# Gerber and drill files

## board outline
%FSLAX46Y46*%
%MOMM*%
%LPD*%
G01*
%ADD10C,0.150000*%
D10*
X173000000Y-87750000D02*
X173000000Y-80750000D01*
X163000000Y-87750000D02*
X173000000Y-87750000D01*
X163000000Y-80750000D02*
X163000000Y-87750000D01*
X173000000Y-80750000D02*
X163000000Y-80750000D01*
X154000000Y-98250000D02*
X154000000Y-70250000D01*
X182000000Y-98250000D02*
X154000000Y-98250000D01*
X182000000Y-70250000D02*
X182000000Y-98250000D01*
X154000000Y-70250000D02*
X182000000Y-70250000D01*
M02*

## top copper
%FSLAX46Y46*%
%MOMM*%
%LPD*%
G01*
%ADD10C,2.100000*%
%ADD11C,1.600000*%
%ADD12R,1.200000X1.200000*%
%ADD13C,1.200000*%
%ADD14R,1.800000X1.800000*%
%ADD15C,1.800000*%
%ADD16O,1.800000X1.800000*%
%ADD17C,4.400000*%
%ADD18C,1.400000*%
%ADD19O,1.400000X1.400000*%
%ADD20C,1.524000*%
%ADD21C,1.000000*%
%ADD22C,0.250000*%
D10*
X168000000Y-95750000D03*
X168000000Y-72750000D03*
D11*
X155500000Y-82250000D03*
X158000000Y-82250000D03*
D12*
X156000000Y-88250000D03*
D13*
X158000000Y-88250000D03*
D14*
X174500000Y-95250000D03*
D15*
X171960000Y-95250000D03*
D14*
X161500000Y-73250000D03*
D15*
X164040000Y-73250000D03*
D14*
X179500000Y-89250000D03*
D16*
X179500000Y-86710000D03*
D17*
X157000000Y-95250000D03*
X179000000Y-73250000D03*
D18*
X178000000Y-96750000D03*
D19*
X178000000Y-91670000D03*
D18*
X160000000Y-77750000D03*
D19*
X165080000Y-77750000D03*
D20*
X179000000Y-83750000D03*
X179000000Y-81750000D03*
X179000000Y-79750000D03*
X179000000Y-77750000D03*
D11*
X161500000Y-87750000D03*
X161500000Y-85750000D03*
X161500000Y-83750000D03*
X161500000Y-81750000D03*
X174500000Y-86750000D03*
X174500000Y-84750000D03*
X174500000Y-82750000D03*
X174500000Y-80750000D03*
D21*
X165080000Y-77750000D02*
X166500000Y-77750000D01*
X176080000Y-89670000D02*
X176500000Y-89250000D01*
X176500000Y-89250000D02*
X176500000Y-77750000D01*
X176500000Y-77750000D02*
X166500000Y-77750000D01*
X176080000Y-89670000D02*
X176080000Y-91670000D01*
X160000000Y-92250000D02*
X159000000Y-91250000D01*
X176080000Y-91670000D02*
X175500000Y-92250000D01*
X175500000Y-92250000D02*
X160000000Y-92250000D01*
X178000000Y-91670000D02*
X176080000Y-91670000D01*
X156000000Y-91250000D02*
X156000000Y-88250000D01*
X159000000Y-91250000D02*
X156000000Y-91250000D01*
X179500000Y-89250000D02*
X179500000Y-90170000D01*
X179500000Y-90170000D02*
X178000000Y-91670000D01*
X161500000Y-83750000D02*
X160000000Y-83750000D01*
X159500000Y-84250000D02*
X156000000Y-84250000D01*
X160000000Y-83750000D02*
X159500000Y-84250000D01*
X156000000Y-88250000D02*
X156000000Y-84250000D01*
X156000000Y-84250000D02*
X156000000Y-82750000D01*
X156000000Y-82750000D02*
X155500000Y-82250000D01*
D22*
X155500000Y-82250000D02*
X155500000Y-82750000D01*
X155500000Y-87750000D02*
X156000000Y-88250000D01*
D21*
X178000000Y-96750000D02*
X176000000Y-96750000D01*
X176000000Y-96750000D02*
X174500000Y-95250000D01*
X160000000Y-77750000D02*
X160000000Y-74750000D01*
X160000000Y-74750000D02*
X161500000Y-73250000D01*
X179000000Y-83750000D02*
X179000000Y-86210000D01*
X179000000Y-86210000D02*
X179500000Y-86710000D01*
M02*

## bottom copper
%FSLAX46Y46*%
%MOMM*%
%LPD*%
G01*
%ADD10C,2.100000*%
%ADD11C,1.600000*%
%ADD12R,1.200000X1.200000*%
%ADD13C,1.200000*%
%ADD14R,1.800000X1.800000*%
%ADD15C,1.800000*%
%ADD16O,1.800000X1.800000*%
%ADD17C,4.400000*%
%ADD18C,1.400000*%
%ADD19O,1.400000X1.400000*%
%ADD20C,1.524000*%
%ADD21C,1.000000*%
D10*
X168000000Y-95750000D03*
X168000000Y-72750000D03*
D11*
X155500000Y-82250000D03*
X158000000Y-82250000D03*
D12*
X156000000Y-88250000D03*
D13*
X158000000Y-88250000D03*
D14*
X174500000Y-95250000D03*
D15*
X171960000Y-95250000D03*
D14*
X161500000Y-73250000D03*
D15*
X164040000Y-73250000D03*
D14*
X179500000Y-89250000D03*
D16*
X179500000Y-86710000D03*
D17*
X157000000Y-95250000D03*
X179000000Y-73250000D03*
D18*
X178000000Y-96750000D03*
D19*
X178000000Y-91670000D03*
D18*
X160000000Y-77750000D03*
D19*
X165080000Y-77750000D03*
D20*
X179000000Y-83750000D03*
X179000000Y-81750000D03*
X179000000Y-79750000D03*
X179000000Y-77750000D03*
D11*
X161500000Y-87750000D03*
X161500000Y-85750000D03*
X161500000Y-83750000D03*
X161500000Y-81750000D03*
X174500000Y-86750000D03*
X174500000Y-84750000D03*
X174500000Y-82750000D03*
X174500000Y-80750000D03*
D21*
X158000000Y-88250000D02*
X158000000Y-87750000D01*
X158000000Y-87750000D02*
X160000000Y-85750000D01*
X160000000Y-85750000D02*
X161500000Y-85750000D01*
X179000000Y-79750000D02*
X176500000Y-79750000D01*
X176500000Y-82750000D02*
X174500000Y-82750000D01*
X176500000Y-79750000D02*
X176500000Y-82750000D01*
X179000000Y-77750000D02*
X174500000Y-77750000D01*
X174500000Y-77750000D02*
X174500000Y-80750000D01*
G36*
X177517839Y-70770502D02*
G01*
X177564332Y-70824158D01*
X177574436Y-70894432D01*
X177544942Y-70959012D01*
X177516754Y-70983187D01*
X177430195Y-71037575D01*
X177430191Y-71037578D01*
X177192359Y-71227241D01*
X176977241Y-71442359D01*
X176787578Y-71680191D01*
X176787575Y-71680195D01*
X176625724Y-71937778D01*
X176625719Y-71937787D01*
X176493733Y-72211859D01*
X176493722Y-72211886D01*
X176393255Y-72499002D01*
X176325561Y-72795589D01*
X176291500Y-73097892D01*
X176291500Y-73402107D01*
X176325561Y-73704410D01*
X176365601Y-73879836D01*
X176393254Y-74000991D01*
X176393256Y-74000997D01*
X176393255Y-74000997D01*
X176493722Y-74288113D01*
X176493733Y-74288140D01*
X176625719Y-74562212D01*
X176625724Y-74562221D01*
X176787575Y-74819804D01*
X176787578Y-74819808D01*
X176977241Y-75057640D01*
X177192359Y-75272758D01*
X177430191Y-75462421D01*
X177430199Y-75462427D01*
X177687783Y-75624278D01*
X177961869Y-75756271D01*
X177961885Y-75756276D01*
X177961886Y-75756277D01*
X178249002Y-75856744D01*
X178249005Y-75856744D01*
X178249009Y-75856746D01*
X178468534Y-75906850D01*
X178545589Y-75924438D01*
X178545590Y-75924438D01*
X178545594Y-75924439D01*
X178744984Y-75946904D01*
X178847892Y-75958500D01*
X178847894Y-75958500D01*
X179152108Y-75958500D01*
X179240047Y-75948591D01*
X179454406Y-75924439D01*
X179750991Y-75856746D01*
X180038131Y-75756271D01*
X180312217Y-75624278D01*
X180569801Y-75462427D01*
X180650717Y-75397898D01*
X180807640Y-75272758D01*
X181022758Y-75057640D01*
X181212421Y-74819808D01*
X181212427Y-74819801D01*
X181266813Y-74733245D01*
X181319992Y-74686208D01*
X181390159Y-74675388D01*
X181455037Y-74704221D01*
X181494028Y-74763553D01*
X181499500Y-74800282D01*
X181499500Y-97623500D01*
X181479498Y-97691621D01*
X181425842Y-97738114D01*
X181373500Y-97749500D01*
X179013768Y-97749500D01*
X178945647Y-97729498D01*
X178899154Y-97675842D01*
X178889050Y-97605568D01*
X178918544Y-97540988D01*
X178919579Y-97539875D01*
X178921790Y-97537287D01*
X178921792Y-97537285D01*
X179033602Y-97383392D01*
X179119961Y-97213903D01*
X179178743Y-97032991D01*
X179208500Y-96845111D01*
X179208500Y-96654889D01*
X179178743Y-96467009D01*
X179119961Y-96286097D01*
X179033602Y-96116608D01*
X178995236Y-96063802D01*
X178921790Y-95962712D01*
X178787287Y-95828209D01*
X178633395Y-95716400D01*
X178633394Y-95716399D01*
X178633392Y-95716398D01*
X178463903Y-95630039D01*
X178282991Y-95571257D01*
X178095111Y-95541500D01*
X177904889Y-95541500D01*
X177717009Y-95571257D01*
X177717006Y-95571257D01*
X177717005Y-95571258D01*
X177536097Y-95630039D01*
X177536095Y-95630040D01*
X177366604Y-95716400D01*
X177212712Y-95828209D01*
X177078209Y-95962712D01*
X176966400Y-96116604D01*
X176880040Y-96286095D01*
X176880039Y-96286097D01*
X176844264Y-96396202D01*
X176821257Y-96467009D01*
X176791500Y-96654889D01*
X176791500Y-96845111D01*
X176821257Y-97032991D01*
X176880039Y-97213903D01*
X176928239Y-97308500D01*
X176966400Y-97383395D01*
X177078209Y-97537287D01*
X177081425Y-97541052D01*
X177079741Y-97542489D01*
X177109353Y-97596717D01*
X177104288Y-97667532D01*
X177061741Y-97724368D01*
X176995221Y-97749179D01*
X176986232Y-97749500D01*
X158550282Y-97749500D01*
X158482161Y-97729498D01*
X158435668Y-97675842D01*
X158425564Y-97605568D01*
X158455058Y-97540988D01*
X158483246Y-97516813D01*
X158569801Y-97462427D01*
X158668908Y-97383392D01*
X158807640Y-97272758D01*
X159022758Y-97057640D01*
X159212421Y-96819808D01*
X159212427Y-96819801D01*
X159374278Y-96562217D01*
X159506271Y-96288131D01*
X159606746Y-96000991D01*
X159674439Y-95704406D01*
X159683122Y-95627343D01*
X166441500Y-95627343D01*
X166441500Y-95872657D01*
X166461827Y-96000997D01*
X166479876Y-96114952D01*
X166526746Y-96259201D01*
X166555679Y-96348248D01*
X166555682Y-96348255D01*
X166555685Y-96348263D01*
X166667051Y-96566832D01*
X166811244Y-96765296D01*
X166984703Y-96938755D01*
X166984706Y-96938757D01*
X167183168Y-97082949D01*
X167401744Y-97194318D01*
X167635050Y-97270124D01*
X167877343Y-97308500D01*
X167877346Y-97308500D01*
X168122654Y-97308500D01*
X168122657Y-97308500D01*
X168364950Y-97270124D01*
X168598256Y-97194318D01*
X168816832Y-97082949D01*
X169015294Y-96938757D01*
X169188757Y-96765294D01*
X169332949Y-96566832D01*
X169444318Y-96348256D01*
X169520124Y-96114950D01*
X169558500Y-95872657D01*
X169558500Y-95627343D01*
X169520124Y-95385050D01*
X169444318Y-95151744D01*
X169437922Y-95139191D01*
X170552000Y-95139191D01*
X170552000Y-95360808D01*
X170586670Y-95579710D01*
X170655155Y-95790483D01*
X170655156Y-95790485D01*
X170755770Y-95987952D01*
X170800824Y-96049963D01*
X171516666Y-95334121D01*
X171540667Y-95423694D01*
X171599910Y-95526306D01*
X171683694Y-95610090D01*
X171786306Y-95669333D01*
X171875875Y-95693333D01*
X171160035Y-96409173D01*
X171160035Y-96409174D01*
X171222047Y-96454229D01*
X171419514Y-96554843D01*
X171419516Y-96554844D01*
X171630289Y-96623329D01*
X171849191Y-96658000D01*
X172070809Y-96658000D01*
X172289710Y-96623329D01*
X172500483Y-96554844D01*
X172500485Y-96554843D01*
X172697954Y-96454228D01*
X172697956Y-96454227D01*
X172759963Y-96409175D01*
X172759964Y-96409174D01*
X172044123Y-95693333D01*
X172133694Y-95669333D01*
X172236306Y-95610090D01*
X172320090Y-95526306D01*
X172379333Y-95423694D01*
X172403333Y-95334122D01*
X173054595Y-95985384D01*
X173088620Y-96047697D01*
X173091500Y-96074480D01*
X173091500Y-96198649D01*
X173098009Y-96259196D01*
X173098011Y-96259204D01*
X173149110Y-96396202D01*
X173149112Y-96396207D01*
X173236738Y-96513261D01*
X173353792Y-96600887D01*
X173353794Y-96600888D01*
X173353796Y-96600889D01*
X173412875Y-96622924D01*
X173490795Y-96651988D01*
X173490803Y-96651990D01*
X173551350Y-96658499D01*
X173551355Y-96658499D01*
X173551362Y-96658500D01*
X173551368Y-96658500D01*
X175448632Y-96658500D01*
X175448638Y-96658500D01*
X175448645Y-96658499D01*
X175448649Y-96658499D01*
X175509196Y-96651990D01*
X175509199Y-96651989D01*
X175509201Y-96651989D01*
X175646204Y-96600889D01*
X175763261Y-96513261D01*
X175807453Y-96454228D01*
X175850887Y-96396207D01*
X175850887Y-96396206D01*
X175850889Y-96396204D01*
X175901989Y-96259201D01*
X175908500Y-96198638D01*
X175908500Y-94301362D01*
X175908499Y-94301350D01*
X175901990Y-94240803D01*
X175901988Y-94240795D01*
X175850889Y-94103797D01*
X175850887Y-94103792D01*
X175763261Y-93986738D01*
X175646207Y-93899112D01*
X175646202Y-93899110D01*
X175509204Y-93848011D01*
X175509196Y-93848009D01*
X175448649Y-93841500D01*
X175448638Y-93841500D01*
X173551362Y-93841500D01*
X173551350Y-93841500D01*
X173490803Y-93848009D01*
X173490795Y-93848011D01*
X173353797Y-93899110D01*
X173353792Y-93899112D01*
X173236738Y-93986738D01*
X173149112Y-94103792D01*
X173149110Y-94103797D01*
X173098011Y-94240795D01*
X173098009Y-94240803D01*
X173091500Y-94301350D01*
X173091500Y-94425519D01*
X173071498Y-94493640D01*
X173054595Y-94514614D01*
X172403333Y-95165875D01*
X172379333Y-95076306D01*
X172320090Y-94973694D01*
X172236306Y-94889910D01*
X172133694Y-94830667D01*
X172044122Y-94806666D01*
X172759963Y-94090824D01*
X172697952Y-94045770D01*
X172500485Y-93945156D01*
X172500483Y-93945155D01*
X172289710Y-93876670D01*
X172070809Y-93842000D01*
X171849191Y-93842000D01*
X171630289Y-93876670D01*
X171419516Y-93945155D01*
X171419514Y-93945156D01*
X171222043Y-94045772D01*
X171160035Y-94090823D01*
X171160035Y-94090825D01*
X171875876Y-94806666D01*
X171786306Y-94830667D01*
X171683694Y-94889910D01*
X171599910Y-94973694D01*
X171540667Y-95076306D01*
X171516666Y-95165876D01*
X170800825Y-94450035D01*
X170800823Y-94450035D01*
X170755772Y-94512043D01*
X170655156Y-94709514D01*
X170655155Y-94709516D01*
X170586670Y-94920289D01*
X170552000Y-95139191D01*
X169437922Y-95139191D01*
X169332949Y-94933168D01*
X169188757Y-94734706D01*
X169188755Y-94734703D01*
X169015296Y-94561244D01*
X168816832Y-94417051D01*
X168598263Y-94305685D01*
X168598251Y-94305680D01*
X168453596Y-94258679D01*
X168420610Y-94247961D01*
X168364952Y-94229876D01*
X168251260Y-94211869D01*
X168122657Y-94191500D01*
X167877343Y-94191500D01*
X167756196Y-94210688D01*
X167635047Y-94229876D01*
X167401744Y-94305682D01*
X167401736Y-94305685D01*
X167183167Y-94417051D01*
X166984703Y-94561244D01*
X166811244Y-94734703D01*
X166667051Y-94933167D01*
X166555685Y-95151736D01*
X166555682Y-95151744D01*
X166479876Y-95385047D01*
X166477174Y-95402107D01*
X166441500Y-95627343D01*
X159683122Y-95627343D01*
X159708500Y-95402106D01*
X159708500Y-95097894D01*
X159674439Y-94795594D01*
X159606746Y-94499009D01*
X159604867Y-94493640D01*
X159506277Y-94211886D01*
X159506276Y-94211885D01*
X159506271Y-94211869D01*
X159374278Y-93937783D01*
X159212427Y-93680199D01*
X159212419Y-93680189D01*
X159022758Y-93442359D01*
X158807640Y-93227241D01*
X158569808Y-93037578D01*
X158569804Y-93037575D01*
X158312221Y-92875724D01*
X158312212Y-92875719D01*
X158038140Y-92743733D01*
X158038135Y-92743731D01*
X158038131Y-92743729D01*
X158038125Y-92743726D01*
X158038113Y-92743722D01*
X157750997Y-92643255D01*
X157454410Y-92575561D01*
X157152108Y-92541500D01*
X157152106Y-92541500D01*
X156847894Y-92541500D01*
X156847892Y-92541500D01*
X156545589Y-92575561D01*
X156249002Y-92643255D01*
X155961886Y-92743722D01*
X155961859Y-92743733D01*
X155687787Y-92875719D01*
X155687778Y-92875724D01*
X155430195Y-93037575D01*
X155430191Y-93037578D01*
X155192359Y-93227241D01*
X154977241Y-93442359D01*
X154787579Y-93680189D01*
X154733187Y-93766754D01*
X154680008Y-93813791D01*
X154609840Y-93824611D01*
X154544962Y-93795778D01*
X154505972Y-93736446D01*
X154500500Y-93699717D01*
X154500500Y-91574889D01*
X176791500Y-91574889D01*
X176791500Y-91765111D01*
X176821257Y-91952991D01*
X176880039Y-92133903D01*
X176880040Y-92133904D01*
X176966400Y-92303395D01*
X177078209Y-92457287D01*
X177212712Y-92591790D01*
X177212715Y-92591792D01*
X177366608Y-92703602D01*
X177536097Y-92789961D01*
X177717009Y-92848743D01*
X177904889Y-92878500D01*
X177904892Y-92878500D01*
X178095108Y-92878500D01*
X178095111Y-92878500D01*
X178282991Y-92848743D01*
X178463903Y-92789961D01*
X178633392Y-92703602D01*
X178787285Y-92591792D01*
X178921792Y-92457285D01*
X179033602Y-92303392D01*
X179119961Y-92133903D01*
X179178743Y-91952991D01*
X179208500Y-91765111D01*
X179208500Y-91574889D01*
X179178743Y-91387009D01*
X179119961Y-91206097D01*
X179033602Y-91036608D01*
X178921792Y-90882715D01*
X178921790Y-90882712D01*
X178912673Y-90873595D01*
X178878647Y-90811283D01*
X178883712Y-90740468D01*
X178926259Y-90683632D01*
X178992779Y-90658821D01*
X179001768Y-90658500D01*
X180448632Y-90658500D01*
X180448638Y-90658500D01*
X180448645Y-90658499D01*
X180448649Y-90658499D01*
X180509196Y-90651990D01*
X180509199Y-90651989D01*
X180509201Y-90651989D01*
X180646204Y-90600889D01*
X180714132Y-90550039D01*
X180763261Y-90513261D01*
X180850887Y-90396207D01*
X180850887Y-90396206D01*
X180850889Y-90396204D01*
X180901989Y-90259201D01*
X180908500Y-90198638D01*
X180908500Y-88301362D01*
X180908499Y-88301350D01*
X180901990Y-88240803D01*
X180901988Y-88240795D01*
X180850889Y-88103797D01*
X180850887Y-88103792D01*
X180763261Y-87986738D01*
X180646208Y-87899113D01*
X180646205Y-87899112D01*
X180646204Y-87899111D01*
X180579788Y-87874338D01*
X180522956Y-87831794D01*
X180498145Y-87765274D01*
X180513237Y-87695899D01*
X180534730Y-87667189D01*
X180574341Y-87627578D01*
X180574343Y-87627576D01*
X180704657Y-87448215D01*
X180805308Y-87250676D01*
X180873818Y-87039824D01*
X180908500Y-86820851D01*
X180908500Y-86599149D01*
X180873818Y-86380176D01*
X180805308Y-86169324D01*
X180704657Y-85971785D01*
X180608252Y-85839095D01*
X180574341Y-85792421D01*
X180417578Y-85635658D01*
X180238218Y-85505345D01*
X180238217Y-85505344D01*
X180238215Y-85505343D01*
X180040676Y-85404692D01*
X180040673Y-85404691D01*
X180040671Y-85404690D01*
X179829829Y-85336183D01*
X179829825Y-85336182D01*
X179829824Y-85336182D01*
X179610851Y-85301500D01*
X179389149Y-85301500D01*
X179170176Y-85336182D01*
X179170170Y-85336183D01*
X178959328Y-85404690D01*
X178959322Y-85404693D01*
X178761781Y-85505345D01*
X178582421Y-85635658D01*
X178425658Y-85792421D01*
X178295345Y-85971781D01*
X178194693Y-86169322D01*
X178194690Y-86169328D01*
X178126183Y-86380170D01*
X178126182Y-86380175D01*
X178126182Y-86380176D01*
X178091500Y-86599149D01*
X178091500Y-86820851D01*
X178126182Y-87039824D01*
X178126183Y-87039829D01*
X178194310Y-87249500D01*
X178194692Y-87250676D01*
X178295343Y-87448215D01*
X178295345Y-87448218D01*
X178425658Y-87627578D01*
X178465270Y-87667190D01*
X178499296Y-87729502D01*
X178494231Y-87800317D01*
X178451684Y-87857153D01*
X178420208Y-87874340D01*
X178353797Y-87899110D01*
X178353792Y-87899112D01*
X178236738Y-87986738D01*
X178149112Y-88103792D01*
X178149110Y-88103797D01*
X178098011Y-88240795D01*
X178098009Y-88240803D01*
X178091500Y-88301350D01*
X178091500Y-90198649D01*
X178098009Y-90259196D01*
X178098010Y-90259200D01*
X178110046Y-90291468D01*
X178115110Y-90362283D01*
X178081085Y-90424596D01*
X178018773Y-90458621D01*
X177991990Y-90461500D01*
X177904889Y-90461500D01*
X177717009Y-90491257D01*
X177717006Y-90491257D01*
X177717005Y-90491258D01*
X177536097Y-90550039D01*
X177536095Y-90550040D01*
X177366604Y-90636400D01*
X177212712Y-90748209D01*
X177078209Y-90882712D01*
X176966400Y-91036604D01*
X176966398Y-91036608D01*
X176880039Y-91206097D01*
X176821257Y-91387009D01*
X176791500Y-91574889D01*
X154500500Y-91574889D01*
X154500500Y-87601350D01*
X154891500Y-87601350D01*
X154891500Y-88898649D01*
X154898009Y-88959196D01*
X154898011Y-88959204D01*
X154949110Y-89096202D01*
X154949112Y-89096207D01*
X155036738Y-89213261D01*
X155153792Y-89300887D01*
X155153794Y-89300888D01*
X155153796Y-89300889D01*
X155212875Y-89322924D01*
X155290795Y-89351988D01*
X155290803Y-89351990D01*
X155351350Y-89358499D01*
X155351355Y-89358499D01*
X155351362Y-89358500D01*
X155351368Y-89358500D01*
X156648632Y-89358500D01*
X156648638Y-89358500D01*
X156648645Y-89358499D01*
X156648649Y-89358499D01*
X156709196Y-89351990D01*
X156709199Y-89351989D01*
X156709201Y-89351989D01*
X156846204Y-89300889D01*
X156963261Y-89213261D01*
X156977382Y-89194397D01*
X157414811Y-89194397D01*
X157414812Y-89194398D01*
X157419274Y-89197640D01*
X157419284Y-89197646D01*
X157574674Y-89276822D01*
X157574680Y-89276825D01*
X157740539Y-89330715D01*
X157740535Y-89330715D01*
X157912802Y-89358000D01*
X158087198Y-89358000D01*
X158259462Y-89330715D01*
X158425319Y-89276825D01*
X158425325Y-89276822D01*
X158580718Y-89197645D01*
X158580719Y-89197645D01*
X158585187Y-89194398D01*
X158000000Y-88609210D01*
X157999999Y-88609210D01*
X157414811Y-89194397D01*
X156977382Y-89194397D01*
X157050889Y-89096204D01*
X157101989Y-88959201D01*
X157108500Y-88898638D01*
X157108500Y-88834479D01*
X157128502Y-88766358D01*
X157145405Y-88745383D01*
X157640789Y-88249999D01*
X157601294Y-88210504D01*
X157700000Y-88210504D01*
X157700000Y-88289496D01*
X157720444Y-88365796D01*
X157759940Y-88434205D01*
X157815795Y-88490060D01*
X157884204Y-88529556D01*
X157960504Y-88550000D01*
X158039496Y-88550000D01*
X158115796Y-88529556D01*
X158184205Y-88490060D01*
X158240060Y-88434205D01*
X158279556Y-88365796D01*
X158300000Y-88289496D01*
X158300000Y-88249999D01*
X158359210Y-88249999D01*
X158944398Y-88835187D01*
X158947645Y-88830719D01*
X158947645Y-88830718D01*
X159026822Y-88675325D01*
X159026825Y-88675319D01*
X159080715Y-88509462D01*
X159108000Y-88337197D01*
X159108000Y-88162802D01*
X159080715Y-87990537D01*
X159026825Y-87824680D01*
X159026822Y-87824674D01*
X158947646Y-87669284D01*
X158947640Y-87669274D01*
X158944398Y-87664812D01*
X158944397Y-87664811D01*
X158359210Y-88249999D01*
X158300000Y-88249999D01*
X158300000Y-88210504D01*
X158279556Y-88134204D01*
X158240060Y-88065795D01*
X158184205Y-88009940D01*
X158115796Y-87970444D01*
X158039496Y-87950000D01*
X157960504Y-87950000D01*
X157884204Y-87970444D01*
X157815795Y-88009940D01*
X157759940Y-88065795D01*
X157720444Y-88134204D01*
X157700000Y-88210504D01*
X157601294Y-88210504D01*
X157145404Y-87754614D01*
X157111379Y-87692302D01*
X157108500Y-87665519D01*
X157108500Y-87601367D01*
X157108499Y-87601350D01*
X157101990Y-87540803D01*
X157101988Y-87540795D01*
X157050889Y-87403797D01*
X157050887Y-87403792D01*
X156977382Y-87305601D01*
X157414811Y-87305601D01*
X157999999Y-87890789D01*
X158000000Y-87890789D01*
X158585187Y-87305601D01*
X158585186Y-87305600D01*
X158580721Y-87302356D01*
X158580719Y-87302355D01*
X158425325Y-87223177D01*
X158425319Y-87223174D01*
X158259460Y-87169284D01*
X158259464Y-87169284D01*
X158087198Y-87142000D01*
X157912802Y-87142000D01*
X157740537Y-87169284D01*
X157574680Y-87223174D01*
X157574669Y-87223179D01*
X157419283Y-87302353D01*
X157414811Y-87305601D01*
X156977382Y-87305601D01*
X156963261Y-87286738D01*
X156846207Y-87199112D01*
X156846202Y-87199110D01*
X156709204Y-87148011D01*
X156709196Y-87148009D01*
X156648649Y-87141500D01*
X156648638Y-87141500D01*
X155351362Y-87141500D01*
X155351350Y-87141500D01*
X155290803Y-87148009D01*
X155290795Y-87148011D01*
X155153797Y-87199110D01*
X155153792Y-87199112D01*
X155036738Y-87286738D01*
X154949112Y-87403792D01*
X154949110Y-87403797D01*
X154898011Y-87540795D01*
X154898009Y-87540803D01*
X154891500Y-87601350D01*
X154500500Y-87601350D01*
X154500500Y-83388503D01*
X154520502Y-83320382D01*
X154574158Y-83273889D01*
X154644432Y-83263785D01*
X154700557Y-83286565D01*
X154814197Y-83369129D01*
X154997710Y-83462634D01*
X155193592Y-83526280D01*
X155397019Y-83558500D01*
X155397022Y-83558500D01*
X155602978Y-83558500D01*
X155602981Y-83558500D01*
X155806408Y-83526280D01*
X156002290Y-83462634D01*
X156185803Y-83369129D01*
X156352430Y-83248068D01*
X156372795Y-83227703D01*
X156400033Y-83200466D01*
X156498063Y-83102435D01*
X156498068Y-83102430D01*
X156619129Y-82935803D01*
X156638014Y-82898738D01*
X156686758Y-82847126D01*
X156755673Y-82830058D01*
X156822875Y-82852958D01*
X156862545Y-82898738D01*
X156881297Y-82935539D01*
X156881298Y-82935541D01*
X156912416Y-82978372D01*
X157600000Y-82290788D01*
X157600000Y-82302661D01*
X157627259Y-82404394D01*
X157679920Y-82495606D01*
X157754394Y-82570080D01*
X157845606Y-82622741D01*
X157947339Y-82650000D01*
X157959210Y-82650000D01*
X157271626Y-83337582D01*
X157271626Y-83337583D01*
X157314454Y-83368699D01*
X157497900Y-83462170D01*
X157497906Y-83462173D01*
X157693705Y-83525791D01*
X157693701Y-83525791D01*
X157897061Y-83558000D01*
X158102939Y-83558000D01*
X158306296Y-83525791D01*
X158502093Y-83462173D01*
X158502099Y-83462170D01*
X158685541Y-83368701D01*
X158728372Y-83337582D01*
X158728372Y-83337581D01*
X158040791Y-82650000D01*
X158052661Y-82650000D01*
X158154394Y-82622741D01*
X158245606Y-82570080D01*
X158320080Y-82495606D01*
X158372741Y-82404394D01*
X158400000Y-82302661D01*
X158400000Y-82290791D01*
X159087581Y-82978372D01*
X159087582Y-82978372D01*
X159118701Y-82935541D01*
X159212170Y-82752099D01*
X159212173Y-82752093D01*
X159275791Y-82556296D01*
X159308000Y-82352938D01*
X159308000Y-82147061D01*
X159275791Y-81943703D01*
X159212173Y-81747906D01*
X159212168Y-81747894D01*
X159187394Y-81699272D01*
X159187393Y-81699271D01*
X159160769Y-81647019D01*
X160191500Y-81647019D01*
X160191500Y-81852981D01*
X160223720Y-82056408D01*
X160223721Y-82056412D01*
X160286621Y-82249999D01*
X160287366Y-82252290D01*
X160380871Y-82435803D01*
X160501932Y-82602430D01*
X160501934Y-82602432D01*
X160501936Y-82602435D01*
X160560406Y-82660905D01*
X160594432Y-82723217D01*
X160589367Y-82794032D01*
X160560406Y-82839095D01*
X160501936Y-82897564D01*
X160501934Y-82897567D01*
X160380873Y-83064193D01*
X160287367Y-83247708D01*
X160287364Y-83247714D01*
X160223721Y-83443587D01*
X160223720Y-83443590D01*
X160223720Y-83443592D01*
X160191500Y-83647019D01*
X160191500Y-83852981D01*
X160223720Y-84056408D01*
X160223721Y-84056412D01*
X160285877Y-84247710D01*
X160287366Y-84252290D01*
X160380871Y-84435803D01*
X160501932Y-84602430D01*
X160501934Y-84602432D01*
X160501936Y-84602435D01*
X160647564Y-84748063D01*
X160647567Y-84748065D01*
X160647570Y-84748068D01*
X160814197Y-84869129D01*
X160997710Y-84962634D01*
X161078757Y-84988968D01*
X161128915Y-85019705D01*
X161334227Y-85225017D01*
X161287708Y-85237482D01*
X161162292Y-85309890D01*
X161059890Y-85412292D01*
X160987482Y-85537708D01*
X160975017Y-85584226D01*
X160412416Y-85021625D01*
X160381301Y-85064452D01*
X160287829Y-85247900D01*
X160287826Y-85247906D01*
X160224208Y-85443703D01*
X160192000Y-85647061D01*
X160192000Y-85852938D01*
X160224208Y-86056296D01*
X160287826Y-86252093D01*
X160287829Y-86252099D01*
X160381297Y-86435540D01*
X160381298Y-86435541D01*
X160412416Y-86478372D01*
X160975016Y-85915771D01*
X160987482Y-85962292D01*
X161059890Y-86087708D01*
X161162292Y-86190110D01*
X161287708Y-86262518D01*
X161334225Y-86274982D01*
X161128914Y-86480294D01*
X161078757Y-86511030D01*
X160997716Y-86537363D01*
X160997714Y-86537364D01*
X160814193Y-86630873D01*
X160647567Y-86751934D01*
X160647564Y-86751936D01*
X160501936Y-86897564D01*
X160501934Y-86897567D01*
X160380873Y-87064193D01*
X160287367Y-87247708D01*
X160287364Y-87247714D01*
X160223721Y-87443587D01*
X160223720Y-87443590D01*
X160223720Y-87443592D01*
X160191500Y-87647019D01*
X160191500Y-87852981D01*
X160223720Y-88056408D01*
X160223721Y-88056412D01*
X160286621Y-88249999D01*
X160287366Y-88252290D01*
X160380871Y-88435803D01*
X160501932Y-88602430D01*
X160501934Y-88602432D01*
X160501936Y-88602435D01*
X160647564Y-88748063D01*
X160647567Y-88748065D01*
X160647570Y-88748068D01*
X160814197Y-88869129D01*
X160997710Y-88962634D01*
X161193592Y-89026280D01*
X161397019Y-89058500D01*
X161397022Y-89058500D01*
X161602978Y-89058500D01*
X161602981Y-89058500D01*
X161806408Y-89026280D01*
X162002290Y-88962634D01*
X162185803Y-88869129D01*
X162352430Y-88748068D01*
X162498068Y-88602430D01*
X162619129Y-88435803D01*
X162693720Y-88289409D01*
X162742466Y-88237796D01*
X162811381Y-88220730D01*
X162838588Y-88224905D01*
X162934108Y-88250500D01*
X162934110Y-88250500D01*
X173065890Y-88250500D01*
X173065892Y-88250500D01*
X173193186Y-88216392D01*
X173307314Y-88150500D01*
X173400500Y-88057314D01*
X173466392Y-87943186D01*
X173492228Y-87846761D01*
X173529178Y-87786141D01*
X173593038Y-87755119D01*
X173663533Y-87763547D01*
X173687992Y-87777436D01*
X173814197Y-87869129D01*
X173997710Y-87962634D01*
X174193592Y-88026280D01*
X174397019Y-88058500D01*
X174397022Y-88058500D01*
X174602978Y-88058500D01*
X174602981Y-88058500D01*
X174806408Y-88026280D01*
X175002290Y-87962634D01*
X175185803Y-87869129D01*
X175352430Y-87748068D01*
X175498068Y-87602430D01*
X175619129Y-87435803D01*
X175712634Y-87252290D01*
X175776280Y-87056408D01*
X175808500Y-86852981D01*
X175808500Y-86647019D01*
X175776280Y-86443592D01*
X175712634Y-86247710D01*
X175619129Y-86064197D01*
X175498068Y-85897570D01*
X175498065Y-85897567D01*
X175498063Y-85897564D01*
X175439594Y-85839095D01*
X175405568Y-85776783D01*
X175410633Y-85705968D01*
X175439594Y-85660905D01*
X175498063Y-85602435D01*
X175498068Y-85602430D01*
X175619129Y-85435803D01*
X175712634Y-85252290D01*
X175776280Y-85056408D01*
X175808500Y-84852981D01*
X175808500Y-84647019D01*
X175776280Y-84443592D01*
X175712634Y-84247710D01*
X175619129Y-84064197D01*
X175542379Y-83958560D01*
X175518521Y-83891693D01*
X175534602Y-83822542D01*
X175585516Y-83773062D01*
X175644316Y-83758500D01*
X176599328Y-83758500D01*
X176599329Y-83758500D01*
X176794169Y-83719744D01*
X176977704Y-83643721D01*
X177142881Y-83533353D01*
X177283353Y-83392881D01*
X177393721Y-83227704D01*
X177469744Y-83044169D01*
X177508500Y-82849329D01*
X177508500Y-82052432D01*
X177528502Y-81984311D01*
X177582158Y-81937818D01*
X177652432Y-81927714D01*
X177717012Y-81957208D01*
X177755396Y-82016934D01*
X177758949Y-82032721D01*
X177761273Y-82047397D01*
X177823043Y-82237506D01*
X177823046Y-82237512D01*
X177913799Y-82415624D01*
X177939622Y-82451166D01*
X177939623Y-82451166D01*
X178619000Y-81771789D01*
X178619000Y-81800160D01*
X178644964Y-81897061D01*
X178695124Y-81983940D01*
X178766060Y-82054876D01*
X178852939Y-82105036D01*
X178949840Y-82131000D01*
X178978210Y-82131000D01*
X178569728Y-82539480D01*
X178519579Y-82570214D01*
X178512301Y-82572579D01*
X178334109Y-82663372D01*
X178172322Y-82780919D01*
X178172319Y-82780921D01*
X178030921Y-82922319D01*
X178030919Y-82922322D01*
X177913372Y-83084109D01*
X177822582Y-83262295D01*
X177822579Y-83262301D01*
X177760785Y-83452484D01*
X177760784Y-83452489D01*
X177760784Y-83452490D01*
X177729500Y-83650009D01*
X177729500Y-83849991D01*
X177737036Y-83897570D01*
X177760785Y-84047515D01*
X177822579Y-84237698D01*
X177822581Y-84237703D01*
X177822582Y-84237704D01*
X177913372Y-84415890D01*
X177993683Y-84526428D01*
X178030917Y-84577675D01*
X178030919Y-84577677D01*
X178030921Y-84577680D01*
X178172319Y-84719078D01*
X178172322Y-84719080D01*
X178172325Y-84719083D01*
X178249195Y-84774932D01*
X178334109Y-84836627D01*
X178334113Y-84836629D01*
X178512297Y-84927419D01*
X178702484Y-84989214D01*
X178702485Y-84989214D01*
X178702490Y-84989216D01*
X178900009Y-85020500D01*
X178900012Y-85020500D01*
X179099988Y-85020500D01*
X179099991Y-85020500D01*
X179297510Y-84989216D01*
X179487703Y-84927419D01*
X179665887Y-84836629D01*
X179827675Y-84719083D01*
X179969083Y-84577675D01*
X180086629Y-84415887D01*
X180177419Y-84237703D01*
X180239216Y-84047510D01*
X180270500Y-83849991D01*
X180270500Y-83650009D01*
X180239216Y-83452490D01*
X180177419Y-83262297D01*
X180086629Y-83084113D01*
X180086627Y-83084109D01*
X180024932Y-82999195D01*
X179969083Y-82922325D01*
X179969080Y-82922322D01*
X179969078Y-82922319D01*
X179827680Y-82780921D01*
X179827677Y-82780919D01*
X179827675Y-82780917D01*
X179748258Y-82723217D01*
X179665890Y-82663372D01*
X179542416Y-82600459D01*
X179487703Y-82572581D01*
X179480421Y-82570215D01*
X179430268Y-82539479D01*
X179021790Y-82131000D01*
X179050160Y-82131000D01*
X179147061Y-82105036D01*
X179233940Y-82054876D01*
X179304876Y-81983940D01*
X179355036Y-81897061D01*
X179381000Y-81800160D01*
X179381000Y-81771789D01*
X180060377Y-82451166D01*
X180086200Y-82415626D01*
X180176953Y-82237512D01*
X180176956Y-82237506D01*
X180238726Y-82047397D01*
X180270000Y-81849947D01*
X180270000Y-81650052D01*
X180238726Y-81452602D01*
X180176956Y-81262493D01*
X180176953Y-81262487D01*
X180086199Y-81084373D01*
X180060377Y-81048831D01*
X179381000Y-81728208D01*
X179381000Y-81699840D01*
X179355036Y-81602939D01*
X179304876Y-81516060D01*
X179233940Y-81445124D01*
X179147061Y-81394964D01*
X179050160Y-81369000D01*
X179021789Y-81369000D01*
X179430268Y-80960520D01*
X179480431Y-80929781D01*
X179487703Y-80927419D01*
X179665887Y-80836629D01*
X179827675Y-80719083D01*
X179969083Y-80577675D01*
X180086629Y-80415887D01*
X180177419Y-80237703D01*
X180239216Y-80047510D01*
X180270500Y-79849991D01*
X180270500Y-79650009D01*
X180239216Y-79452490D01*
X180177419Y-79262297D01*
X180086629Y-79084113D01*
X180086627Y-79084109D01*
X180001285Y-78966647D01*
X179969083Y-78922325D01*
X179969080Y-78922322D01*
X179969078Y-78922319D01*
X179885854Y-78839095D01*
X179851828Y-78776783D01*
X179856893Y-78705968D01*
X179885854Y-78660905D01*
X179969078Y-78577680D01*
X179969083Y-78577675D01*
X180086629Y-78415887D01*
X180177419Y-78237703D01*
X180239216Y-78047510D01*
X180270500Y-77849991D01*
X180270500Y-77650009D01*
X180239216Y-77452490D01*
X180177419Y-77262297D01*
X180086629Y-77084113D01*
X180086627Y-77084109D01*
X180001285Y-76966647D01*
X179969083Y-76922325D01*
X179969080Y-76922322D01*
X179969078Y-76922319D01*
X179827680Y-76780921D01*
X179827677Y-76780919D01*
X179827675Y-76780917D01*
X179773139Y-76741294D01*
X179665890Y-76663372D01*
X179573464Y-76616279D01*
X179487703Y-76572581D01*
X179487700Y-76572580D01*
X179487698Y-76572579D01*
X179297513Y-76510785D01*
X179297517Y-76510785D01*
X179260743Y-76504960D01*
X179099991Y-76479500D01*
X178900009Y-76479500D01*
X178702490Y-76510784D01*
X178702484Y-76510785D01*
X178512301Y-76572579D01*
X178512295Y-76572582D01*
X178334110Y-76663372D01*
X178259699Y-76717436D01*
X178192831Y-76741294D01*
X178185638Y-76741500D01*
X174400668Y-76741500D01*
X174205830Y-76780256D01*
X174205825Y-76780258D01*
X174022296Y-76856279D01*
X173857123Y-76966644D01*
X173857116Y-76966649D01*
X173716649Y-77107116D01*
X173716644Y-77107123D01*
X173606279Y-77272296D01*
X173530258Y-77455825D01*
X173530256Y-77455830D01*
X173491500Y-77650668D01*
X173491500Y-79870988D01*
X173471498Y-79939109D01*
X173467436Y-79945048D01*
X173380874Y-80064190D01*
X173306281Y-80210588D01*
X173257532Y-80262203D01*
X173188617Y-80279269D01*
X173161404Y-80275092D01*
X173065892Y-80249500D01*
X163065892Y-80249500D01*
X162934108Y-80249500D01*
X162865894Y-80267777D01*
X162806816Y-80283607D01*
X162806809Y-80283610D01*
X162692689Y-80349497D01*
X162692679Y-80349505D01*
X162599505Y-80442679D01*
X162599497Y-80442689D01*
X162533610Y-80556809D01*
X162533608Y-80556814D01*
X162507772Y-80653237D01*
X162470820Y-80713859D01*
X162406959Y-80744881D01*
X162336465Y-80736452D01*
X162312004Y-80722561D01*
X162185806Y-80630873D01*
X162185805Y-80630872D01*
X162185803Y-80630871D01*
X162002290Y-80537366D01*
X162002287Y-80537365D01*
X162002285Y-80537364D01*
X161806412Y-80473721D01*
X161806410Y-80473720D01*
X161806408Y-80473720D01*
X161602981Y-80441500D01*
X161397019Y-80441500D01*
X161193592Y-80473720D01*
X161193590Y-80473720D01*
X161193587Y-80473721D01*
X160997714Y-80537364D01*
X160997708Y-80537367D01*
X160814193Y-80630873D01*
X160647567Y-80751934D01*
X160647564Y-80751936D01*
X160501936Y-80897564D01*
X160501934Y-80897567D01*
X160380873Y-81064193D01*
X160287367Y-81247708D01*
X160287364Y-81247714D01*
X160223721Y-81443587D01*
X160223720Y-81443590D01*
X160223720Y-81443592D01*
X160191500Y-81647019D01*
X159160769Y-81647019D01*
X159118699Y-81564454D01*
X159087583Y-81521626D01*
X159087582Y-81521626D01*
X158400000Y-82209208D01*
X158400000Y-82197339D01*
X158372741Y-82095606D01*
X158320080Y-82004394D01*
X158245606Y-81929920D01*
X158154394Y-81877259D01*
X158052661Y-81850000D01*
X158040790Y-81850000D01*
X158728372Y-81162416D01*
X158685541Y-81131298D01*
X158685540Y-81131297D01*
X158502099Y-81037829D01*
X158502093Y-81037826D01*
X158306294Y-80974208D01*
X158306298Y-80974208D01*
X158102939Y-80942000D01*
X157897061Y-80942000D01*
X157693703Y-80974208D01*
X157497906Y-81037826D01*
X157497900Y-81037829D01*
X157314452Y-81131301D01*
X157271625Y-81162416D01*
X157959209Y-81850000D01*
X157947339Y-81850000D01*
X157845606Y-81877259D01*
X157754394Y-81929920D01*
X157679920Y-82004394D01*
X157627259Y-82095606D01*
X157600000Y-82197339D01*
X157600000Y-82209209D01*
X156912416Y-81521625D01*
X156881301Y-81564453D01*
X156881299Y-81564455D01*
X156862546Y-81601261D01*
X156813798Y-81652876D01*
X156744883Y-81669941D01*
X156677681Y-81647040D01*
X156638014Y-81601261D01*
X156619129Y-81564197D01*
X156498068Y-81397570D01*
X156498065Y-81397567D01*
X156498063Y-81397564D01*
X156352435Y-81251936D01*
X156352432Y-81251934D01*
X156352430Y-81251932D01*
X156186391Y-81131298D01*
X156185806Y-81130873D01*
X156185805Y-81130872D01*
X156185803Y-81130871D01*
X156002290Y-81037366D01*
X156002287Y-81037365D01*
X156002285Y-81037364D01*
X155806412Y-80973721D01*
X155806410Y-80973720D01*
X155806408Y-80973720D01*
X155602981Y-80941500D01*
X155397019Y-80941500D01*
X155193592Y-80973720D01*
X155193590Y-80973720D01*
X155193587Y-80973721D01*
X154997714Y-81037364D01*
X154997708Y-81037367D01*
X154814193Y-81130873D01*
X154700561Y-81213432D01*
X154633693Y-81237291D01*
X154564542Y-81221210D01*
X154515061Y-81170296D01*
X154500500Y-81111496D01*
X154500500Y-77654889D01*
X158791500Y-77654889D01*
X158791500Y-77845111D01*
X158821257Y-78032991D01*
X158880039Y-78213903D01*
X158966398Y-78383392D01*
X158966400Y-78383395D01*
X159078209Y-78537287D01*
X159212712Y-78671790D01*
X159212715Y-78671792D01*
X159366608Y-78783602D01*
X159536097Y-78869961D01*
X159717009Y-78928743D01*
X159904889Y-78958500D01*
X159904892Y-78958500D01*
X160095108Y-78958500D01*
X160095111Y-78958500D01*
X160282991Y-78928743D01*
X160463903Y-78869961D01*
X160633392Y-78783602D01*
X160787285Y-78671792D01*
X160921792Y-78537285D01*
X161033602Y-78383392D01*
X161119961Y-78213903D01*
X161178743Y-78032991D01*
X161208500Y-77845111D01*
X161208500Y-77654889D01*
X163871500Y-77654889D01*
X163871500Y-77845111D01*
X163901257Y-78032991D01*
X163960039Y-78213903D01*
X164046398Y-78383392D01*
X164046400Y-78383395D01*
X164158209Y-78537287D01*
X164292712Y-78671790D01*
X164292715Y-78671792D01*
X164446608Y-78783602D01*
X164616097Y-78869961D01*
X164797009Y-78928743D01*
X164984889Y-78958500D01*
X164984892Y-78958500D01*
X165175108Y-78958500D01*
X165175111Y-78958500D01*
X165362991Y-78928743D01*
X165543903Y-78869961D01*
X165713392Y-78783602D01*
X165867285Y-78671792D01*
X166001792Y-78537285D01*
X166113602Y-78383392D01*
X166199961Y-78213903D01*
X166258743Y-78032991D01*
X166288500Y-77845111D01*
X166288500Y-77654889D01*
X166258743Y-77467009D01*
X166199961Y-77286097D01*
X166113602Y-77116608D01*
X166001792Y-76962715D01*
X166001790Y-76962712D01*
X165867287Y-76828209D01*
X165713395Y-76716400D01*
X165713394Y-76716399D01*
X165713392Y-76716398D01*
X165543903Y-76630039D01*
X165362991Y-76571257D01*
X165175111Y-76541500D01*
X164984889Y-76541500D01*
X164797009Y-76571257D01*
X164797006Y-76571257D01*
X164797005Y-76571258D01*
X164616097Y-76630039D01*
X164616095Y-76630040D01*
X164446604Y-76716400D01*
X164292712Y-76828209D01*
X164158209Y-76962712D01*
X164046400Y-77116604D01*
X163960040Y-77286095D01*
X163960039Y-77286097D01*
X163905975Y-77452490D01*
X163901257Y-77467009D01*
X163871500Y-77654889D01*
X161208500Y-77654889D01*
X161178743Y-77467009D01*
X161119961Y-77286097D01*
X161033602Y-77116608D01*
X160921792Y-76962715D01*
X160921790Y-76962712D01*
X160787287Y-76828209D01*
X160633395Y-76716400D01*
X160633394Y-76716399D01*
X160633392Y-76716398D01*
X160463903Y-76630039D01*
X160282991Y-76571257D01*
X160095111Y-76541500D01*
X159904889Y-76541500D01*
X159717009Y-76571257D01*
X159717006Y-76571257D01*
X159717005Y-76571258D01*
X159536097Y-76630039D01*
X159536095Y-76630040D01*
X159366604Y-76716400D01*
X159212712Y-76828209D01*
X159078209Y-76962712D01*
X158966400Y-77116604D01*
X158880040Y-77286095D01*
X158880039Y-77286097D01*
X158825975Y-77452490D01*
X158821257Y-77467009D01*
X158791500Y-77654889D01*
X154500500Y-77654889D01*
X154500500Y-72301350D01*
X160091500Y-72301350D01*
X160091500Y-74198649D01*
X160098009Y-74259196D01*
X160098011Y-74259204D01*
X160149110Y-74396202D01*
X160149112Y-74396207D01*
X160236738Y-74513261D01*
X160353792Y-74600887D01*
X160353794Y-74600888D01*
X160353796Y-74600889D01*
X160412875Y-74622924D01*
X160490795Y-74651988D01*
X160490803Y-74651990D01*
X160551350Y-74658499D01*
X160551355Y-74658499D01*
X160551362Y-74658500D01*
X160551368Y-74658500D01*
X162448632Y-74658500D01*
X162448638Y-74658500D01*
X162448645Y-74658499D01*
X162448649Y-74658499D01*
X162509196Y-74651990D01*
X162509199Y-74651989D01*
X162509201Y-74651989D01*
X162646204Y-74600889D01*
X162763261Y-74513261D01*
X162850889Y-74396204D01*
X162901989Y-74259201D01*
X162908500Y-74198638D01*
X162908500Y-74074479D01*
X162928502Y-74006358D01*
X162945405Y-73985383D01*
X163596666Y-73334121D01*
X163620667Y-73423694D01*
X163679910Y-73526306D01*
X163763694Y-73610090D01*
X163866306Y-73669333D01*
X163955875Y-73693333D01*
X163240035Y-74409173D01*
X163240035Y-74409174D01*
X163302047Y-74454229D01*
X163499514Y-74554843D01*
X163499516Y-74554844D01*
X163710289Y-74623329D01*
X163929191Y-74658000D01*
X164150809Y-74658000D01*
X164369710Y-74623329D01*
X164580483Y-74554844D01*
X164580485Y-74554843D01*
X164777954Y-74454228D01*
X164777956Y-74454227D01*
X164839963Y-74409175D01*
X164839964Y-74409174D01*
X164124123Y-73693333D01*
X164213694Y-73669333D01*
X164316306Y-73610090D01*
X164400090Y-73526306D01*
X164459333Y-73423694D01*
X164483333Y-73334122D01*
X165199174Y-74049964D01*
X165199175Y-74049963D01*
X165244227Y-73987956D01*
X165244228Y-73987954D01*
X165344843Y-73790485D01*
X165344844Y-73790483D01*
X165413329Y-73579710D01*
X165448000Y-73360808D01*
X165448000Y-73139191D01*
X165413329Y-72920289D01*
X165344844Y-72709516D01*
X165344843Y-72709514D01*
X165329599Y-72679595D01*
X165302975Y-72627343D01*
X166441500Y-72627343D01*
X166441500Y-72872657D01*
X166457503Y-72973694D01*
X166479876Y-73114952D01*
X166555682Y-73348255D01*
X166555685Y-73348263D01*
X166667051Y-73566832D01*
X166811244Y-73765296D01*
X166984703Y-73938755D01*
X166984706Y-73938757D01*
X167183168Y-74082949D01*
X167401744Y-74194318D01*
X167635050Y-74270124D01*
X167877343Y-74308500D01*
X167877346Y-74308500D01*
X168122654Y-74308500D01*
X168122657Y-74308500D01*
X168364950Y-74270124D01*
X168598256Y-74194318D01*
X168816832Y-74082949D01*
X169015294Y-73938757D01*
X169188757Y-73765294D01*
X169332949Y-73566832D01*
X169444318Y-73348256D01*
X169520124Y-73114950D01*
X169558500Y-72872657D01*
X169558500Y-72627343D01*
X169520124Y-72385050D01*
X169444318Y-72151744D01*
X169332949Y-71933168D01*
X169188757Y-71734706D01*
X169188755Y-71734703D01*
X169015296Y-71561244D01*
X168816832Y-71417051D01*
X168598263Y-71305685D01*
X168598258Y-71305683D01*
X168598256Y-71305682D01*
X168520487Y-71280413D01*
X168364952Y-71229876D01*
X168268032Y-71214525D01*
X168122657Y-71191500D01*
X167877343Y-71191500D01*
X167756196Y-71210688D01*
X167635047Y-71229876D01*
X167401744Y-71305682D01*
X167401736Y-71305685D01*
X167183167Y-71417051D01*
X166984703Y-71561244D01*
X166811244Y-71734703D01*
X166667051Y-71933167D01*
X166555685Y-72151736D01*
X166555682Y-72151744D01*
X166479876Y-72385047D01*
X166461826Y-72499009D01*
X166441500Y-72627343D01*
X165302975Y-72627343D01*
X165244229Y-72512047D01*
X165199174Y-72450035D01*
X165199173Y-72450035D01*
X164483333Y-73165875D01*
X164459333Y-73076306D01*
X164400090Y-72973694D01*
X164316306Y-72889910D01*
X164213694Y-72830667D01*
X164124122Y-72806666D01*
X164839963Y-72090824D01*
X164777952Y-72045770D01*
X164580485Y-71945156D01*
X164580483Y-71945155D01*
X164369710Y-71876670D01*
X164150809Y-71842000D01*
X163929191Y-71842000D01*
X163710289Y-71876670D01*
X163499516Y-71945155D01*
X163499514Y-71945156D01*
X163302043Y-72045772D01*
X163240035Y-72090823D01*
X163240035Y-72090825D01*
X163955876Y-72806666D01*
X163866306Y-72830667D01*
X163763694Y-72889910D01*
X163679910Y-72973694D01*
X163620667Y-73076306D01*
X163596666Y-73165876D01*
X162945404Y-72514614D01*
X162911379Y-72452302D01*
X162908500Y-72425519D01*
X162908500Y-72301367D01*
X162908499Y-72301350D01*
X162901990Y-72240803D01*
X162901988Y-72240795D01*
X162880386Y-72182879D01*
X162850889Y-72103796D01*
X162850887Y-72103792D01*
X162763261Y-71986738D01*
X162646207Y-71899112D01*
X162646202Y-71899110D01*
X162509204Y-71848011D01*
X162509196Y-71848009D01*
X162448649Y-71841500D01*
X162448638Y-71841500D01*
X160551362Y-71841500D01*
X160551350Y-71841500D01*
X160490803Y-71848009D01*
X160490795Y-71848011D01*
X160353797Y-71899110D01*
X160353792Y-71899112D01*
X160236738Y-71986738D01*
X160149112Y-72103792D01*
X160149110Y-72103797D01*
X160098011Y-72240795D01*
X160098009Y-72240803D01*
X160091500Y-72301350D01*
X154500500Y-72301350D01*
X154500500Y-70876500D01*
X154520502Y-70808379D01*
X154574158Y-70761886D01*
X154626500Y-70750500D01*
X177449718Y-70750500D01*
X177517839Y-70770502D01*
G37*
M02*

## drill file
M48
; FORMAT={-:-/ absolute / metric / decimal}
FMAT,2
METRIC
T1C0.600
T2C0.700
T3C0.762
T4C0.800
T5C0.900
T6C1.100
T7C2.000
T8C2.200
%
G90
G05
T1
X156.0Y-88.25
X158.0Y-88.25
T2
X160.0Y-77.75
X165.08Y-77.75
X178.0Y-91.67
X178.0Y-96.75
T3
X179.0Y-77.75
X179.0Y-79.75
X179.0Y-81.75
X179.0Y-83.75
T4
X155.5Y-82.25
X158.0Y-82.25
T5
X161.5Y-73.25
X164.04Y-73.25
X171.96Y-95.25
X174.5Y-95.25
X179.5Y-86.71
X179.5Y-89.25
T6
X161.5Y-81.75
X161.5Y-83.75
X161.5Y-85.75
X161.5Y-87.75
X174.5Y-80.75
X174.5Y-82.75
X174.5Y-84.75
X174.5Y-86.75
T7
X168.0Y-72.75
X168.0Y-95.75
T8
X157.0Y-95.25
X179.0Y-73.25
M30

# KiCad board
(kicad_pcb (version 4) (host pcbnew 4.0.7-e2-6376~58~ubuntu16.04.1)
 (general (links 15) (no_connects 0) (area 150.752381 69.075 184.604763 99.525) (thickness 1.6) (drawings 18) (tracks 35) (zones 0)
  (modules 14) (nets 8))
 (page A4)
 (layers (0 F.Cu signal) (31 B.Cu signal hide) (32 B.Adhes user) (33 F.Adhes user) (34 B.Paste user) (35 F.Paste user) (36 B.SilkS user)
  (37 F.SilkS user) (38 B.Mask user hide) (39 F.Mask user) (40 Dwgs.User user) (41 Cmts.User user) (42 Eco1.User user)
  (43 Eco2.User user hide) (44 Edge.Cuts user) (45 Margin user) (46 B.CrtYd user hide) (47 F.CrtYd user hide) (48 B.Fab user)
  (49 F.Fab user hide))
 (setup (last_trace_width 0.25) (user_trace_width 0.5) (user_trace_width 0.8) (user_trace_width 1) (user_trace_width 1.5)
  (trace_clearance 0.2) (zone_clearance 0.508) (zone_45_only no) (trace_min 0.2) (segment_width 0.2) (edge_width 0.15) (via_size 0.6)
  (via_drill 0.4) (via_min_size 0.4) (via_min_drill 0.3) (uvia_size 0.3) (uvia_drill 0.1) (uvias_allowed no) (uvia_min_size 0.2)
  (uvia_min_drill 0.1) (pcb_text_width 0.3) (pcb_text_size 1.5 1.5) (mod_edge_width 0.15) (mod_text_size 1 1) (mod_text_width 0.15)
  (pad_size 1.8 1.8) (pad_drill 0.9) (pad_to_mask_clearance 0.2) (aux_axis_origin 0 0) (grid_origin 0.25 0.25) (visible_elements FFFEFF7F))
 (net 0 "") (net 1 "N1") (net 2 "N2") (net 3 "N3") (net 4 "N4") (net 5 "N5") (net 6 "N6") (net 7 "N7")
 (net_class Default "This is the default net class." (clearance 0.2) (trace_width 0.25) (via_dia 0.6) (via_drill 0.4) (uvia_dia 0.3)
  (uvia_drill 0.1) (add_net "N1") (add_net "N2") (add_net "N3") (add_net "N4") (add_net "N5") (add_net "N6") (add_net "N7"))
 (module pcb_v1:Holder (layer F.Cu) (at 168 81.75)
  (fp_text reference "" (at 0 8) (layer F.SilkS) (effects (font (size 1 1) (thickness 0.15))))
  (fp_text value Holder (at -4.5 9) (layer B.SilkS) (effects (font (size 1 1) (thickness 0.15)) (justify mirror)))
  (pad 1 thru_hole circle (at 0 14) (size 2.1 2.1) (drill 2) (layers *.Cu *.Mask))
  (pad 2 thru_hole circle (at 0 -9) (size 2.1 2.1) (drill 2) (layers *.Cu *.Mask)))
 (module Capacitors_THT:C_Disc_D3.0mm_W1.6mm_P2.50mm (layer F.Cu) (at 155.5 82.25)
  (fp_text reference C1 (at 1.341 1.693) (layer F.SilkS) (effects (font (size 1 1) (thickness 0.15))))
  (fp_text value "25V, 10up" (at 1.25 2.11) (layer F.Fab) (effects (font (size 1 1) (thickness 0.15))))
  (pad 1 thru_hole circle (at 0 0) (size 1.6 1.6) (drill 0.8) (layers *.Cu *.Mask) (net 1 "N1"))
  (pad 2 thru_hole circle (at 2.5 0) (size 1.6 1.6) (drill 0.8) (layers *.Cu *.Mask) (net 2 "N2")))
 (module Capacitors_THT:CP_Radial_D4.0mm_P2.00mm (layer F.Cu) (at 156 88.25)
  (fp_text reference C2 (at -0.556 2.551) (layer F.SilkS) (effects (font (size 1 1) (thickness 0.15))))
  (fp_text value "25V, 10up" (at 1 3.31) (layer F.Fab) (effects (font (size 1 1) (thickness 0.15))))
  (pad 1 thru_hole rect (at 0 0) (size 1.2 1.2) (drill 0.6) (layers *.Cu *.Mask) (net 1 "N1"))
  (pad 2 thru_hole circle (at 2 0) (size 1.2 1.2) (drill 0.6) (layers *.Cu *.Mask) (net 2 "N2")))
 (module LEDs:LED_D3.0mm (layer F.Cu) (at 174.5 95.25 180)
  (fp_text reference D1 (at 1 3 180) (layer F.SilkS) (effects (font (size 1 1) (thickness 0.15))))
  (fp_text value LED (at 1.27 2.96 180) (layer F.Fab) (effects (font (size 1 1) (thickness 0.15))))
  (pad 1 thru_hole rect (at 0 0 180) (size 1.8 1.8) (drill 0.9) (layers *.Cu *.Mask) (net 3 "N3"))
  (pad 2 thru_hole circle (at 2.54 0 180) (size 1.8 1.8) (drill 0.9) (layers *.Cu *.Mask) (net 2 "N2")))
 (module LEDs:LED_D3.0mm (layer F.Cu) (at 161.5 73.25)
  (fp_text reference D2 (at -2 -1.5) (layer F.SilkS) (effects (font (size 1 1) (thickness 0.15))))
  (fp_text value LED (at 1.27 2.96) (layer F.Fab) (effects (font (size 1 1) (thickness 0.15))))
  (pad 1 thru_hole rect (at 0 0) (size 1.8 1.8) (drill 0.9) (layers *.Cu *.Mask) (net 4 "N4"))
  (pad 2 thru_hole circle (at 2.54 0) (size 1.8 1.8) (drill 0.9) (layers *.Cu *.Mask) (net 2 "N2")))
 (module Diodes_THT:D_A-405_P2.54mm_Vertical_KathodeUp (layer F.Cu) (at 179.5 89.25 90)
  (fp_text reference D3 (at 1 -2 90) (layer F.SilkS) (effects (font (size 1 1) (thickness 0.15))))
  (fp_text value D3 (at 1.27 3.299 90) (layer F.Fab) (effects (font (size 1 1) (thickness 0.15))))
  (pad 1 thru_hole rect (at 0 0 90) (size 1.8 1.8) (drill 0.9) (layers *.Cu *.Mask) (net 1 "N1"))
  (pad 2 thru_hole oval (at 2.54 0 90) (size 1.8 1.8) (drill 0.9) (layers *.Cu *.Mask) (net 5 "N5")))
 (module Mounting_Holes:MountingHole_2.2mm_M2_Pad (layer F.Cu) (at 157 95.25)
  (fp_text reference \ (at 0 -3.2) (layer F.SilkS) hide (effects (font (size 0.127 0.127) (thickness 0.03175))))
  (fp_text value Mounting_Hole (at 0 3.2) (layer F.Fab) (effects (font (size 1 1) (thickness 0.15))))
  (pad 1 thru_hole circle (at 0 0) (size 4.4 4.4) (drill 2.2) (layers *.Cu *.Mask)))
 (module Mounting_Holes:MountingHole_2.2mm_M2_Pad (layer F.Cu) (at 179 73.25)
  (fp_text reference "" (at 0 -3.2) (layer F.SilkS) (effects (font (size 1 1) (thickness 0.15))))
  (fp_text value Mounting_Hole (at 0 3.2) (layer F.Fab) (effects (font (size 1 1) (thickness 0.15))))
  (pad 1 thru_hole circle (at 0 0) (size 4.4 4.4) (drill 2.2) (layers *.Cu *.Mask)))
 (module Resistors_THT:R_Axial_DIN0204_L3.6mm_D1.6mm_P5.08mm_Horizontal (layer F.Cu) (at 178 96.75 90)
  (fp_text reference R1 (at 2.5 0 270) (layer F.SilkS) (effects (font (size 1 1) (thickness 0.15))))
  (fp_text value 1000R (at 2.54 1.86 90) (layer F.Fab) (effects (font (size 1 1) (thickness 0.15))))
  (pad 1 thru_hole circle (at 0 0 90) (size 1.4 1.4) (drill 0.7) (layers *.Cu *.Mask) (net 3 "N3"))
  (pad 2 thru_hole oval (at 5.08 0 90) (size 1.4 1.4) (drill 0.7) (layers *.Cu *.Mask) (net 1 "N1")))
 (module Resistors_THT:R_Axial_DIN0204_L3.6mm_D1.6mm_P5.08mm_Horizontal (layer F.Cu) (at 160 77.75)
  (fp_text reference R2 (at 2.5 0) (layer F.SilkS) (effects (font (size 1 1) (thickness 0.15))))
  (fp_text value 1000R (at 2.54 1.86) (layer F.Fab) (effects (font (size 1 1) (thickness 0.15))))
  (pad 1 thru_hole circle (at 0 0) (size 1.4 1.4) (drill 0.7) (layers *.Cu *.Mask) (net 4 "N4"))
  (pad 2 thru_hole oval (at 5.08 0) (size 1.4 1.4) (drill 0.7) (layers *.Cu *.Mask) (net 1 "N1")))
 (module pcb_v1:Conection (layer F.Cu) (at 179 79.75 90)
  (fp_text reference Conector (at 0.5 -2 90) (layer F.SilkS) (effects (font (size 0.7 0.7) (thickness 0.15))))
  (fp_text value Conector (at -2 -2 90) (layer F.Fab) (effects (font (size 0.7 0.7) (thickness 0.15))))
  (pad 1 thru_hole circle (at -4 0 90) (size 1.524 1.524) (drill 0.762) (layers *.Cu *.Mask) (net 5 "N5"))
  (pad 2 thru_hole circle (at -2 0 90) (size 1.524 1.524) (drill 0.762) (layers *.Cu *.Mask) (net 2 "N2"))
  (pad 3 thru_hole circle (at 0 0 90) (size 1.524 1.524) (drill 0.762) (layers *.Cu *.Mask) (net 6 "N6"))
  (pad 4 thru_hole circle (at 2 0 90) (size 1.524 1.524) (drill 0.762) (layers *.Cu *.Mask) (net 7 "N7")))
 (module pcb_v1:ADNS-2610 (layer F.Cu) (at 168 86.75)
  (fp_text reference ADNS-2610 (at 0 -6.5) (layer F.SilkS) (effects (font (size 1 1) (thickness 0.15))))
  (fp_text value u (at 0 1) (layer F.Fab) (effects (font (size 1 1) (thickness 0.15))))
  (pad 8 thru_hole circle (at -6.5 1) (size 1.6 1.6) (drill 1.1) (layers *.Cu *.Mask))
  (pad 7 thru_hole circle (at -6.5 -1) (size 1.6 1.6) (drill 1.1) (layers *.Cu *.Mask) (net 2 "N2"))
  (pad 6 thru_hole circle (at -6.5 -3) (size 1.6 1.6) (drill 1.1) (layers *.Cu *.Mask) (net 1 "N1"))
  (pad 5 thru_hole circle (at -6.5 -5) (size 1.6 1.6) (drill 1.1) (layers *.Cu *.Mask))
  (pad 1 thru_hole circle (at 6.5 0) (size 1.6 1.6) (drill 1.1) (layers *.Cu *.Mask))
  (pad 2 thru_hole circle (at 6.5 -2) (size 1.6 1.6) (drill 1.1) (layers *.Cu *.Mask))
  (pad 3 thru_hole circle (at 6.5 -4) (size 1.6 1.6) (drill 1.1) (layers *.Cu *.Mask) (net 6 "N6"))
  (pad 4 thru_hole circle (at 6.5 -6) (size 1.6 1.6) (drill 1.1) (layers *.Cu *.Mask) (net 7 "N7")))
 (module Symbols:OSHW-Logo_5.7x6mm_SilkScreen (layer F.Cu) (at 162.75 94.25)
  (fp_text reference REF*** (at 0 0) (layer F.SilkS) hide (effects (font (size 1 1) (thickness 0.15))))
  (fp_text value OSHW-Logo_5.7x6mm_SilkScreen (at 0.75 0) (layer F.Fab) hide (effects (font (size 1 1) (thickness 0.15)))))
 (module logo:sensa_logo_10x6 (layer F.Cu) (at 156.841 75.942 90)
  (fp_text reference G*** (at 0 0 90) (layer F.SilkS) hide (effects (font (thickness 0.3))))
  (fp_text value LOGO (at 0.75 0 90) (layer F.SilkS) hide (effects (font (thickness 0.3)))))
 (gr_line (start 173 87.75) (end 173 80.75) (angle 90) (layer Edge.Cuts) (width 0.15))
 (gr_line (start 163 87.75) (end 173 87.75) (angle 90) (layer Edge.Cuts) (width 0.15))
 (gr_line (start 163 80.75) (end 163 87.75) (angle 90) (layer Edge.Cuts) (width 0.15))
 (gr_line (start 173 80.75) (end 163 80.75) (angle 90) (layer Edge.Cuts) (width 0.15))
 (gr_line (start 154 98.25) (end 154 70.25) (angle 90) (layer Edge.Cuts) (width 0.15))
 (gr_line (start 182 98.25) (end 154 98.25) (angle 90) (layer Edge.Cuts) (width 0.15))
 (gr_line (start 182 70.25) (end 182 98.25) (angle 90) (layer Edge.Cuts) (width 0.15))
 (gr_line (start 154 70.25) (end 182 70.25) (angle 90) (layer Edge.Cuts) (width 0.15))
 (segment (start 165.08 77.75) (end 166.5 77.75) (width 1) (layer F.Cu) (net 1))
 (segment (start 176.08 89.67) (end 176.5 89.25) (width 1) (layer F.Cu) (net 1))
 (segment (start 176.5 89.25) (end 176.5 77.75) (width 1) (layer F.Cu) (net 1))
 (segment (start 176.5 77.75) (end 166.5 77.75) (width 1) (layer F.Cu) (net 1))
 (segment (start 176.08 89.67) (end 176.08 91.67) (width 1) (layer F.Cu) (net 1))
 (segment (start 160 92.25) (end 159 91.25) (width 1) (layer F.Cu) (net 1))
 (segment (start 176.08 91.67) (end 175.5 92.25) (width 1) (layer F.Cu) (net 1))
 (segment (start 175.5 92.25) (end 160 92.25) (width 1) (layer F.Cu) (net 1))
 (segment (start 178 91.67) (end 176.08 91.67) (width 1) (layer F.Cu) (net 1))
 (segment (start 156 91.25) (end 156 88.25) (width 1) (layer F.Cu) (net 1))
 (segment (start 159 91.25) (end 156 91.25) (width 1) (layer F.Cu) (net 1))
 (segment (start 179.5 89.25) (end 179.5 90.17) (width 1) (layer F.Cu) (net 1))
 (segment (start 179.5 90.17) (end 178 91.67) (width 1) (layer F.Cu) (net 1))
 (segment (start 161.5 83.75) (end 160 83.75) (width 1) (layer F.Cu) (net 1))
 (segment (start 159.5 84.25) (end 156 84.25) (width 1) (layer F.Cu) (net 1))
 (segment (start 160 83.75) (end 159.5 84.25) (width 1) (layer F.Cu) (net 1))
 (segment (start 156 88.25) (end 156 84.25) (width 1) (layer F.Cu) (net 1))
 (segment (start 156 84.25) (end 156 82.75) (width 1) (layer F.Cu) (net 1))
 (segment (start 156 82.75) (end 155.5 82.25) (width 1) (layer F.Cu) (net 1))
 (segment (start 155.5 82.25) (end 155.5 82.75) (width 0.25) (layer F.Cu) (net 1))
 (segment (start 155.5 87.75) (end 156 88.25) (width 0.25) (layer F.Cu) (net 1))
 (segment (start 158 88.25) (end 158 87.75) (width 1) (layer B.Cu) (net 2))
 (segment (start 158 87.75) (end 160 85.75) (width 1) (layer B.Cu) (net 2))
 (segment (start 160 85.75) (end 161.5 85.75) (width 1) (layer B.Cu) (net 2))
 (segment (start 178 96.75) (end 176 96.75) (width 1) (layer F.Cu) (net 3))
 (segment (start 176 96.75) (end 174.5 95.25) (width 1) (layer F.Cu) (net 3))
 (segment (start 160 77.75) (end 160 74.75) (width 1) (layer F.Cu) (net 4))
 (segment (start 160 74.75) (end 161.5 73.25) (width 1) (layer F.Cu) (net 4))
 (segment (start 179 83.75) (end 179 86.21) (width 1) (layer F.Cu) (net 5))
 (segment (start 179 86.21) (end 179.5 86.71) (width 1) (layer F.Cu) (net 5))
 (segment (start 179 79.75) (end 176.5 79.75) (width 1) (layer B.Cu) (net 6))
 (segment (start 176.5 82.75) (end 174.5 82.75) (width 1) (layer B.Cu) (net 6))
 (segment (start 176.5 79.75) (end 176.5 82.75) (width 1) (layer B.Cu) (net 6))
 (segment (start 179 77.75) (end 174.5 77.75) (width 1) (layer B.Cu) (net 7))
 (segment (start 174.5 77.75) (end 174.5 80.75) (width 1) (layer B.Cu) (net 7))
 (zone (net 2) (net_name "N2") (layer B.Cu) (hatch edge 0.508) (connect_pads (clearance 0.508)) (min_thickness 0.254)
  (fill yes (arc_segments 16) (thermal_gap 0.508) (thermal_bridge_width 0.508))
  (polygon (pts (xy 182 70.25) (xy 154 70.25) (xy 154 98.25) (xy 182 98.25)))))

